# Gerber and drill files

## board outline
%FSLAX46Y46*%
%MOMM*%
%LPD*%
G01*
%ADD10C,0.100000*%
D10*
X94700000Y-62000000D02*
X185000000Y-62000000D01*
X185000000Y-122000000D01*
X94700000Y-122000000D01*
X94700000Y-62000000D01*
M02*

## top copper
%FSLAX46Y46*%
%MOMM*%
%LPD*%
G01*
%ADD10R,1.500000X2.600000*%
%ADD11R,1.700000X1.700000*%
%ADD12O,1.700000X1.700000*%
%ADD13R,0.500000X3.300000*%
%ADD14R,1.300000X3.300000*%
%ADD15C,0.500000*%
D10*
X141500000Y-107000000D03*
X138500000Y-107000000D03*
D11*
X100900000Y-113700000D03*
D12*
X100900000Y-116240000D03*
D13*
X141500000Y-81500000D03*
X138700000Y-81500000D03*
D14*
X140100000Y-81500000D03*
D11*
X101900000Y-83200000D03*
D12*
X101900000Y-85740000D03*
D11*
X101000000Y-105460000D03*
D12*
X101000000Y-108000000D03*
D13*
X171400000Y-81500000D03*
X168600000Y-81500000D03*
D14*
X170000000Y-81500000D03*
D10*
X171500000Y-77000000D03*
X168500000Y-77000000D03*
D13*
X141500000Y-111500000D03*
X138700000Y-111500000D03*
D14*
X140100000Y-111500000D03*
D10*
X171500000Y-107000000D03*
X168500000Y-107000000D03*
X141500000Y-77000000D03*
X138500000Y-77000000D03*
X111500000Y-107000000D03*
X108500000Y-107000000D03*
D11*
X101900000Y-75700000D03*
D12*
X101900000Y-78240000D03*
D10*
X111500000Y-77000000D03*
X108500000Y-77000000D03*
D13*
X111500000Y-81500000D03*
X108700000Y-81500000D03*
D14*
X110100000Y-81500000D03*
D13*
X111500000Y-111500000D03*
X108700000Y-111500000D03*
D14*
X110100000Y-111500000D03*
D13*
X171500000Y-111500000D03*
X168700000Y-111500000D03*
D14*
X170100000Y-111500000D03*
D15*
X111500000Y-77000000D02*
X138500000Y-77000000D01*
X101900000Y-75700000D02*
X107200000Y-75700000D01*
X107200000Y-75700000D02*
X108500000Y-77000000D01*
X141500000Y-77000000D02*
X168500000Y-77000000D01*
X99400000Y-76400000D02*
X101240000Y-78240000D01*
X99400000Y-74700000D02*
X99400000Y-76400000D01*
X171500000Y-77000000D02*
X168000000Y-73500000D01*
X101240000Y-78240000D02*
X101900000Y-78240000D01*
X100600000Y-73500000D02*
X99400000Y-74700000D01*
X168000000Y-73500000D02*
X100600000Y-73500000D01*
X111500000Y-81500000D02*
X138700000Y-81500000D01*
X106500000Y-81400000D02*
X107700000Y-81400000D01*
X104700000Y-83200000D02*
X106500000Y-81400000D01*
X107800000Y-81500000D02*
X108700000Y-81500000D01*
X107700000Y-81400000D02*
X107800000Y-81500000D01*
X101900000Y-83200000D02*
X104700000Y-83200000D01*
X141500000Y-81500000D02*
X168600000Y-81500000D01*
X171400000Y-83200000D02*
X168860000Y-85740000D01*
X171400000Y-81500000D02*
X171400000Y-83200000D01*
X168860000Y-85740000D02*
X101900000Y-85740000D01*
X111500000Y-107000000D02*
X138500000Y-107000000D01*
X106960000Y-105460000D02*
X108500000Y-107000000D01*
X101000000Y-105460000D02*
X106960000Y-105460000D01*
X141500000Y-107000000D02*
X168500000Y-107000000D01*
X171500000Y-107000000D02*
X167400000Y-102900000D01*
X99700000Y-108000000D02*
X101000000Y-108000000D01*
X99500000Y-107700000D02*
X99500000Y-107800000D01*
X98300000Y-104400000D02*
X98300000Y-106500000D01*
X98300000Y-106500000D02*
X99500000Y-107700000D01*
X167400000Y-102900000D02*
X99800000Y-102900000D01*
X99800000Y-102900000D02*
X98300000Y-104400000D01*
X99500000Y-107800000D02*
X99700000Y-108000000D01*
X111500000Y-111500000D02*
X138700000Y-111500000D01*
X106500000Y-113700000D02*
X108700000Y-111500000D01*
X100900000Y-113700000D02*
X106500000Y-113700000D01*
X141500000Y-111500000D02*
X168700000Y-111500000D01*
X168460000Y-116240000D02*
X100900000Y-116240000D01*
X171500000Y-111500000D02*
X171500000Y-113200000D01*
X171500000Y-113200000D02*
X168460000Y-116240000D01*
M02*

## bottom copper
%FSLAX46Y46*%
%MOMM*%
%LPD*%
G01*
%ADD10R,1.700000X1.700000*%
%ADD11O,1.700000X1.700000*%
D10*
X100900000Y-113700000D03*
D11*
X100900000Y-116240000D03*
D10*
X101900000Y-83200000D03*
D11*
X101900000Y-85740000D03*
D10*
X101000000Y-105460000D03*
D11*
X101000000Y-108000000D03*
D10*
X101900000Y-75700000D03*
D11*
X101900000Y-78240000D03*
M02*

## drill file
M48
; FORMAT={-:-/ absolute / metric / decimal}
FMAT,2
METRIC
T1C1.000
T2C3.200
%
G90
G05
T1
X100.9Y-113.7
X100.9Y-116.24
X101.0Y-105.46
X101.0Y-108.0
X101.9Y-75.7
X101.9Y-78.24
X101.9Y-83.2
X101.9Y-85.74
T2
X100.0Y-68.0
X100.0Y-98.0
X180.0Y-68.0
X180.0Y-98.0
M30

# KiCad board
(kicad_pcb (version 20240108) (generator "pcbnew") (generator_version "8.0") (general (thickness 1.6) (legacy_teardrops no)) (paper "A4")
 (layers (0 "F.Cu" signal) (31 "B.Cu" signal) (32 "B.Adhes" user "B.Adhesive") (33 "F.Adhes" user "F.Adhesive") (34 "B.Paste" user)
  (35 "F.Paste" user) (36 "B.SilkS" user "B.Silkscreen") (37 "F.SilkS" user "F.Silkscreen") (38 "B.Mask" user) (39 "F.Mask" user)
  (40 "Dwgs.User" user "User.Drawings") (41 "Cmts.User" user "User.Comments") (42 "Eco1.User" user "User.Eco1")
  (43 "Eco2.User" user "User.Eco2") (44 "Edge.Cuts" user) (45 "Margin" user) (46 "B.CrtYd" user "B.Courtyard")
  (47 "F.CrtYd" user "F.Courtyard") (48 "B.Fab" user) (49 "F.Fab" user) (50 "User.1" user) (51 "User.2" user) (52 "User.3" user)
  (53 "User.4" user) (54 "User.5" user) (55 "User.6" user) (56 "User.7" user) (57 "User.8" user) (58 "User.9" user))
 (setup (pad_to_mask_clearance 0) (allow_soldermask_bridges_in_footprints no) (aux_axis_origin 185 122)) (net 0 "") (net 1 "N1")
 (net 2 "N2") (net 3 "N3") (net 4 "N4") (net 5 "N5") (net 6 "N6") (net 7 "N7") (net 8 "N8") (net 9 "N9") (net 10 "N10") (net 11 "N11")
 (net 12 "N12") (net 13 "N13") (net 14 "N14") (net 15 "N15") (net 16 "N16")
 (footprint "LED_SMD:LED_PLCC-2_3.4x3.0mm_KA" (layer "F.Cu") (at 140 107 180)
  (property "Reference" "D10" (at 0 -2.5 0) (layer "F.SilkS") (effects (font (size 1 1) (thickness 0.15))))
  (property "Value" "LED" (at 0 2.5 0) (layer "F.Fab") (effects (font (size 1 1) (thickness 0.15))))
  (pad "1" smd rect (at -1.5 0 180) (size 1.5 2.6) (layers "F.Cu" "F.Paste" "F.Mask") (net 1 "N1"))
  (pad "2" smd rect (at 1.5 0 180) (size 1.5 2.6) (layers "F.Cu" "F.Paste" "F.Mask") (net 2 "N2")))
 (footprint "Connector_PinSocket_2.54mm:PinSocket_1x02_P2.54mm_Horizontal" (layer "F.Cu") (at 100.9 113.7)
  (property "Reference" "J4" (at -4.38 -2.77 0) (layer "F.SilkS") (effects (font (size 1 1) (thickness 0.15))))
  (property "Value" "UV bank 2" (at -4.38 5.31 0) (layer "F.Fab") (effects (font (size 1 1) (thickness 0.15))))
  (pad "1" thru_hole rect (at 0 0) (size 1.7 1.7) (drill 1) (layers "*.Cu" "*.Mask") (remove_unused_layers no) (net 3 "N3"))
  (pad "2" thru_hole oval (at 0 2.54) (size 1.7 1.7) (drill 1) (layers "*.Cu" "*.Mask") (remove_unused_layers no) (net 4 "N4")))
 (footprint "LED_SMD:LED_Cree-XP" (layer "F.Cu") (at 140.1 81.5 180)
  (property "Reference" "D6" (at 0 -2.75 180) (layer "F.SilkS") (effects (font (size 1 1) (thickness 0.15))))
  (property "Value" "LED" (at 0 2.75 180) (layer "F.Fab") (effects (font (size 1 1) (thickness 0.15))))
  (pad "" smd rect (at 0 -1 180) (size 1.01 0.75) (layers "F.Paste"))
  (pad "" smd rect (at 0 0 180) (size 1.01 0.75) (layers "F.Paste"))
  (pad "" smd rect (at 0 1 180) (size 1.01 0.75) (layers "F.Paste"))
  (pad "1" smd rect (at -1.4 0 180) (size 0.5 3.3) (layers "F.Cu" "F.Paste" "F.Mask") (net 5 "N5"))
  (pad "2" smd rect (at 1.4 0 180) (size 0.5 3.3) (layers "F.Cu" "F.Paste" "F.Mask") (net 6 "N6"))
  (pad "3" smd rect (at 0 0 180) (size 1.3 3.3) (layers "F.Cu" "F.Mask")))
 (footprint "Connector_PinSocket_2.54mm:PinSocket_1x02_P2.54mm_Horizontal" (layer "F.Cu") (at 101.9 83.2)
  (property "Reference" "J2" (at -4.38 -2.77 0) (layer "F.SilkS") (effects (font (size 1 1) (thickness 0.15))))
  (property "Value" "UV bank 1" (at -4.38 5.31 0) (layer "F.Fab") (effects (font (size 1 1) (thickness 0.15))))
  (pad "1" thru_hole rect (at 0 0) (size 1.7 1.7) (drill 1) (layers "*.Cu" "*.Mask") (remove_unused_layers no) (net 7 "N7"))
  (pad "2" thru_hole oval (at 0 2.54) (size 1.7 1.7) (drill 1) (layers "*.Cu" "*.Mask") (remove_unused_layers no) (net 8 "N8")))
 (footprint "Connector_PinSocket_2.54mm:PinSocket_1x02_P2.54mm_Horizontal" (layer "F.Cu") (at 101 105.46)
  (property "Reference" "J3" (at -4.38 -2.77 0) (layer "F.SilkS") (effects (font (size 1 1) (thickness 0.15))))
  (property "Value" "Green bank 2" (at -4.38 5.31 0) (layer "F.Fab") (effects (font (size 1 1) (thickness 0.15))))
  (pad "1" thru_hole rect (at 0 0) (size 1.7 1.7) (drill 1) (layers "*.Cu" "*.Mask") (remove_unused_layers no) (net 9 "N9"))
  (pad "2" thru_hole oval (at 0 2.54) (size 1.7 1.7) (drill 1) (layers "*.Cu" "*.Mask") (remove_unused_layers no) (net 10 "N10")))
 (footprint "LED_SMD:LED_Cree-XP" (layer "F.Cu") (at 170 81.5 180)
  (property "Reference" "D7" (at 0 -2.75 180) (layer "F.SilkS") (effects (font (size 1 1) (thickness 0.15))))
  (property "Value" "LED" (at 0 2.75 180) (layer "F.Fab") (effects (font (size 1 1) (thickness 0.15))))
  (pad "" smd rect (at 0 -1 180) (size 1.01 0.75) (layers "F.Paste"))
  (pad "" smd rect (at 0 0 180) (size 1.01 0.75) (layers "F.Paste"))
  (pad "" smd rect (at 0 1 180) (size 1.01 0.75) (layers "F.Paste"))
  (pad "1" smd rect (at -1.4 0 180) (size 0.5 3.3) (layers "F.Cu" "F.Paste" "F.Mask") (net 8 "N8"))
  (pad "2" smd rect (at 1.4 0 180) (size 0.5 3.3) (layers "F.Cu" "F.Paste" "F.Mask") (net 5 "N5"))
  (pad "3" smd rect (at 0 0 180) (size 1.3 3.3) (layers "F.Cu" "F.Mask")))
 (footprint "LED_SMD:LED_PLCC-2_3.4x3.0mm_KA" (layer "F.Cu") (at 170 77 180)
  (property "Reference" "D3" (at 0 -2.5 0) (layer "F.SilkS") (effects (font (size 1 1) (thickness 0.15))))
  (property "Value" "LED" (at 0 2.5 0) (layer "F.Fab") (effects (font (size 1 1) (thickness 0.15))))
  (pad "1" smd rect (at -1.5 0 180) (size 1.5 2.6) (layers "F.Cu" "F.Paste" "F.Mask") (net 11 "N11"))
  (pad "2" smd rect (at 1.5 0 180) (size 1.5 2.6) (layers "F.Cu" "F.Paste" "F.Mask") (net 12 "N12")))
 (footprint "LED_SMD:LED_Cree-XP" (layer "F.Cu") (at 140.1 111.5 180)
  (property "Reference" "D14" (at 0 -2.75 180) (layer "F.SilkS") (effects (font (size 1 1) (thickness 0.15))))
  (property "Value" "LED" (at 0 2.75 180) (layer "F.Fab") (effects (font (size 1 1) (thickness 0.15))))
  (pad "" smd rect (at 0 -1 180) (size 1.01 0.75) (layers "F.Paste"))
  (pad "" smd rect (at 0 0 180) (size 1.01 0.75) (layers "F.Paste"))
  (pad "" smd rect (at 0 1 180) (size 1.01 0.75) (layers "F.Paste"))
  (pad "1" smd rect (at -1.4 0 180) (size 0.5 3.3) (layers "F.Cu" "F.Paste" "F.Mask") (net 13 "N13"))
  (pad "2" smd rect (at 1.4 0 180) (size 0.5 3.3) (layers "F.Cu" "F.Paste" "F.Mask") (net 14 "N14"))
  (pad "3" smd rect (at 0 0 180) (size 1.3 3.3) (layers "F.Cu" "F.Mask")))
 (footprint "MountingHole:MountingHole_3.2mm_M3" (layer "F.Cu") (at 180 68)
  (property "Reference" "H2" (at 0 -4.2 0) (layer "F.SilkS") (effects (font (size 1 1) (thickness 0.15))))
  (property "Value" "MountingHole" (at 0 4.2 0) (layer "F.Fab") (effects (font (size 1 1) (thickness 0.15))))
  (pad "" np_thru_hole circle (at 0 0) (size 3.2 3.2) (drill 3.2) (layers "*.Cu" "*.Mask")))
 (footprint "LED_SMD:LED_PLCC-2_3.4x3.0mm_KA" (layer "F.Cu") (at 170 107 180)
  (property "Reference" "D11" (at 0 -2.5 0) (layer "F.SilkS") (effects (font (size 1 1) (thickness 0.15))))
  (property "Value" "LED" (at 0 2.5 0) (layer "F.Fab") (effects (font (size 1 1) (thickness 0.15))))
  (pad "1" smd rect (at -1.5 0 180) (size 1.5 2.6) (layers "F.Cu" "F.Paste" "F.Mask") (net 10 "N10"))
  (pad "2" smd rect (at 1.5 0 180) (size 1.5 2.6) (layers "F.Cu" "F.Paste" "F.Mask") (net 1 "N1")))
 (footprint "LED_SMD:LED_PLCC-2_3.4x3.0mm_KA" (layer "F.Cu") (at 140 77 180)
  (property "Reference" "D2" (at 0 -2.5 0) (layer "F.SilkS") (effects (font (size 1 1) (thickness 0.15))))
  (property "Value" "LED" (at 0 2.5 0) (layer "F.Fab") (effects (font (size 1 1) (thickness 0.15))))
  (pad "1" smd rect (at -1.5 0 180) (size 1.5 2.6) (layers "F.Cu" "F.Paste" "F.Mask") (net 12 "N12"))
  (pad "2" smd rect (at 1.5 0 180) (size 1.5 2.6) (layers "F.Cu" "F.Paste" "F.Mask") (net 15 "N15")))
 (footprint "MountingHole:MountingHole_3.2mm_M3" (layer "F.Cu") (at 100 98)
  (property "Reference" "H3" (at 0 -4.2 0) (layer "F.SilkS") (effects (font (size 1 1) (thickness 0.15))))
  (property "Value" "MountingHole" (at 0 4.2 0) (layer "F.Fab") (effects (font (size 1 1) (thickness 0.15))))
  (pad "" np_thru_hole circle (at 0 0) (size 3.2 3.2) (drill 3.2) (layers "*.Cu" "*.Mask")))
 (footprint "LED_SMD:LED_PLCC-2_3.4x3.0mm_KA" (layer "F.Cu") (at 110 107 180)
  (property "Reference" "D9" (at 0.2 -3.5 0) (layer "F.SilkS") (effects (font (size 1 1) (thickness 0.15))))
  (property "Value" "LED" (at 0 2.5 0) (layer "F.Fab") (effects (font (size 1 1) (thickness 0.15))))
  (pad "1" smd rect (at -1.5 0 180) (size 1.5 2.6) (layers "F.Cu" "F.Paste" "F.Mask") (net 2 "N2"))
  (pad "2" smd rect (at 1.5 0 180) (size 1.5 2.6) (layers "F.Cu" "F.Paste" "F.Mask") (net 9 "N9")))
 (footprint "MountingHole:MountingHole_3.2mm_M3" (layer "F.Cu") (at 180 98)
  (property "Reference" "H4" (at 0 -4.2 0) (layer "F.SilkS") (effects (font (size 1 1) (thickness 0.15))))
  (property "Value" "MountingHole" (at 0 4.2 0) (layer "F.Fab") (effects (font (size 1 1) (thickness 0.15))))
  (pad "" np_thru_hole circle (at 0 0) (size 3.2 3.2) (drill 3.2) (layers "*.Cu" "*.Mask")))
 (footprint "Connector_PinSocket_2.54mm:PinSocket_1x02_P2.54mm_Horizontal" (layer "F.Cu") (at 101.9 75.7)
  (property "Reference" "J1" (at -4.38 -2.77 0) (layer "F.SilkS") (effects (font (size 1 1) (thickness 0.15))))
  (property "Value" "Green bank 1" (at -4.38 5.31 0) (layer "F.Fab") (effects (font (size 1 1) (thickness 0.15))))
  (pad "1" thru_hole rect (at 0 0) (size 1.7 1.7) (drill 1) (layers "*.Cu" "*.Mask") (remove_unused_layers no) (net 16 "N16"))
  (pad "2" thru_hole oval (at 0 2.54) (size 1.7 1.7) (drill 1) (layers "*.Cu" "*.Mask") (remove_unused_layers no) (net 11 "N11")))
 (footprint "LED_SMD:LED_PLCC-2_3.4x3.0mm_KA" (layer "F.Cu") (at 110 77 180)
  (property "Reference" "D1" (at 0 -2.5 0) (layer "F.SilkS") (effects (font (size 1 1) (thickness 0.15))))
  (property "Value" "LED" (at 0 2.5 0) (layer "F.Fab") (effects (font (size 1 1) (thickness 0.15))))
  (pad "1" smd rect (at -1.5 0 180) (size 1.5 2.6) (layers "F.Cu" "F.Paste" "F.Mask") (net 15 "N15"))
  (pad "2" smd rect (at 1.5 0 180) (size 1.5 2.6) (layers "F.Cu" "F.Paste" "F.Mask") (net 16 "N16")))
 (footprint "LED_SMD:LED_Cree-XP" (layer "F.Cu") (at 110.1 81.5 180)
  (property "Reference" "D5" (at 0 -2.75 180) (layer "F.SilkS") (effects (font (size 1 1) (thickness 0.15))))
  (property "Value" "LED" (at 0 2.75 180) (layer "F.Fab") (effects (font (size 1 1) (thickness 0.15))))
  (pad "" smd rect (at 0 -1 180) (size 1.01 0.75) (layers "F.Paste"))
  (pad "" smd rect (at 0 0 180) (size 1.01 0.75) (layers "F.Paste"))
  (pad "" smd rect (at 0 1 180) (size 1.01 0.75) (layers "F.Paste"))
  (pad "1" smd rect (at -1.4 0 180) (size 0.5 3.3) (layers "F.Cu" "F.Paste" "F.Mask") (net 6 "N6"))
  (pad "2" smd rect (at 1.4 0 180) (size 0.5 3.3) (layers "F.Cu" "F.Paste" "F.Mask") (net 7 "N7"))
  (pad "3" smd rect (at 0 0 180) (size 1.3 3.3) (layers "F.Cu" "F.Mask")))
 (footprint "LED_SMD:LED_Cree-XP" (layer "F.Cu") (at 110.1 111.5 180)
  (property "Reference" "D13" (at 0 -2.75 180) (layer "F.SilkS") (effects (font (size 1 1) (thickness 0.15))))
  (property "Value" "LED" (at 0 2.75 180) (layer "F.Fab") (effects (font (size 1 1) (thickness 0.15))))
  (pad "" smd rect (at 0 -1 180) (size 1.01 0.75) (layers "F.Paste"))
  (pad "" smd rect (at 0 0 180) (size 1.01 0.75) (layers "F.Paste"))
  (pad "" smd rect (at 0 1 180) (size 1.01 0.75) (layers "F.Paste"))
  (pad "1" smd rect (at -1.4 0 180) (size 0.5 3.3) (layers "F.Cu" "F.Paste" "F.Mask") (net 14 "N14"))
  (pad "2" smd rect (at 1.4 0 180) (size 0.5 3.3) (layers "F.Cu" "F.Paste" "F.Mask") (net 3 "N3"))
  (pad "3" smd rect (at 0 0 180) (size 1.3 3.3) (layers "F.Cu" "F.Mask")))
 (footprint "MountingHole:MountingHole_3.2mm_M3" (layer "F.Cu") (at 100 68)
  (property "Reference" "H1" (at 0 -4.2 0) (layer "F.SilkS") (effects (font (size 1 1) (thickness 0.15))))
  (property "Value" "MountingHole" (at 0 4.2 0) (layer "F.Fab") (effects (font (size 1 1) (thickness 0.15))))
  (pad "" np_thru_hole circle (at 0 0) (size 3.2 3.2) (drill 3.2) (layers "F&B.Cu" "*.Mask")))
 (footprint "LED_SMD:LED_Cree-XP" (layer "F.Cu") (at 170.1 111.5 180)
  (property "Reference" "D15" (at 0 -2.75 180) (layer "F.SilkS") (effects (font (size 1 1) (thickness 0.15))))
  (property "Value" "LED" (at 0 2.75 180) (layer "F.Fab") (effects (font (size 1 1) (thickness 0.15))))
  (pad "" smd rect (at 0 -1 180) (size 1.01 0.75) (layers "F.Paste"))
  (pad "" smd rect (at 0 0 180) (size 1.01 0.75) (layers "F.Paste"))
  (pad "" smd rect (at 0 1 180) (size 1.01 0.75) (layers "F.Paste"))
  (pad "1" smd rect (at -1.4 0 180) (size 0.5 3.3) (layers "F.Cu" "F.Paste" "F.Mask") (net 4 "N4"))
  (pad "2" smd rect (at 1.4 0 180) (size 0.5 3.3) (layers "F.Cu" "F.Paste" "F.Mask") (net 13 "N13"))
  (pad "3" smd rect (at 0 0 180) (size 1.3 3.3) (layers "F.Cu" "F.Mask")))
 (gr_rect (start 94.7 62) (end 185 122) (stroke (width 0.1) (type default)) (fill none) (layer "Edge.Cuts"))
 (segment (start 111.5 77) (end 138.5 77) (width 0.5) (layer "F.Cu") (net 15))
 (segment (start 101.9 75.7) (end 107.2 75.7) (width 0.5) (layer "F.Cu") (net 16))
 (segment (start 107.2 75.7) (end 108.5 77) (width 0.5) (layer "F.Cu") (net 16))
 (segment (start 141.5 77) (end 168.5 77) (width 0.5) (layer "F.Cu") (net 12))
 (segment (start 99.4 76.4) (end 101.24 78.24) (width 0.5) (layer "F.Cu") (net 11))
 (segment (start 99.4 74.7) (end 99.4 76.4) (width 0.5) (layer "F.Cu") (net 11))
 (segment (start 171.5 77) (end 168 73.5) (width 0.5) (layer "F.Cu") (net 11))
 (segment (start 101.24 78.24) (end 101.9 78.24) (width 0.5) (layer "F.Cu") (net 11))
 (segment (start 100.6 73.5) (end 99.4 74.7) (width 0.5) (layer "F.Cu") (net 11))
 (segment (start 168 73.5) (end 100.6 73.5) (width 0.5) (layer "F.Cu") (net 11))
 (segment (start 111.5 81.5) (end 138.7 81.5) (width 0.5) (layer "F.Cu") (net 6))
 (segment (start 106.5 81.4) (end 107.7 81.4) (width 0.5) (layer "F.Cu") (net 7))
 (segment (start 104.7 83.2) (end 106.5 81.4) (width 0.5) (layer "F.Cu") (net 7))
 (segment (start 107.8 81.5) (end 108.7 81.5) (width 0.5) (layer "F.Cu") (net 7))
 (segment (start 107.7 81.4) (end 107.8 81.5) (width 0.5) (layer "F.Cu") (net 7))
 (segment (start 101.9 83.2) (end 104.7 83.2) (width 0.5) (layer "F.Cu") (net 7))
 (segment (start 141.5 81.5) (end 168.6 81.5) (width 0.5) (layer "F.Cu") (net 5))
 (segment (start 171.4 83.2) (end 168.86 85.74) (width 0.5) (layer "F.Cu") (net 8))
 (segment (start 171.4 81.5) (end 171.4 83.2) (width 0.5) (layer "F.Cu") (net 8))
 (segment (start 168.86 85.74) (end 101.9 85.74) (width 0.5) (layer "F.Cu") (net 8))
 (segment (start 111.5 107) (end 138.5 107) (width 0.5) (layer "F.Cu") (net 2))
 (segment (start 106.96 105.46) (end 108.5 107) (width 0.5) (layer "F.Cu") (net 9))
 (segment (start 101 105.46) (end 106.96 105.46) (width 0.5) (layer "F.Cu") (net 9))
 (segment (start 141.5 107) (end 168.5 107) (width 0.5) (layer "F.Cu") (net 1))
 (segment (start 171.5 107) (end 167.4 102.9) (width 0.5) (layer "F.Cu") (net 10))
 (segment (start 99.7 108) (end 101 108) (width 0.5) (layer "F.Cu") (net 10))
 (segment (start 99.5 107.7) (end 99.5 107.8) (width 0.5) (layer "F.Cu") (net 10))
 (segment (start 98.3 104.4) (end 98.3 106.5) (width 0.5) (layer "F.Cu") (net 10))
 (segment (start 98.3 106.5) (end 99.5 107.7) (width 0.5) (layer "F.Cu") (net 10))
 (segment (start 167.4 102.9) (end 99.8 102.9) (width 0.5) (layer "F.Cu") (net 10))
 (segment (start 99.8 102.9) (end 98.3 104.4) (width 0.5) (layer "F.Cu") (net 10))
 (segment (start 99.5 107.8) (end 99.7 108) (width 0.5) (layer "F.Cu") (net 10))
 (segment (start 111.5 111.5) (end 138.7 111.5) (width 0.5) (layer "F.Cu") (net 14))
 (segment (start 106.5 113.7) (end 108.7 111.5) (width 0.5) (layer "F.Cu") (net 3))
 (segment (start 100.9 113.7) (end 106.5 113.7) (width 0.5) (layer "F.Cu") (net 3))
 (segment (start 141.5 111.5) (end 168.7 111.5) (width 0.5) (layer "F.Cu") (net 13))
 (segment (start 168.46 116.24) (end 100.9 116.24) (width 0.5) (layer "F.Cu") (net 4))
 (segment (start 171.5 111.5) (end 171.5 113.2) (width 0.5) (layer "F.Cu") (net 4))
 (segment (start 171.5 113.2) (end 168.46 116.24) (width 0.5) (layer "F.Cu") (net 4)))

